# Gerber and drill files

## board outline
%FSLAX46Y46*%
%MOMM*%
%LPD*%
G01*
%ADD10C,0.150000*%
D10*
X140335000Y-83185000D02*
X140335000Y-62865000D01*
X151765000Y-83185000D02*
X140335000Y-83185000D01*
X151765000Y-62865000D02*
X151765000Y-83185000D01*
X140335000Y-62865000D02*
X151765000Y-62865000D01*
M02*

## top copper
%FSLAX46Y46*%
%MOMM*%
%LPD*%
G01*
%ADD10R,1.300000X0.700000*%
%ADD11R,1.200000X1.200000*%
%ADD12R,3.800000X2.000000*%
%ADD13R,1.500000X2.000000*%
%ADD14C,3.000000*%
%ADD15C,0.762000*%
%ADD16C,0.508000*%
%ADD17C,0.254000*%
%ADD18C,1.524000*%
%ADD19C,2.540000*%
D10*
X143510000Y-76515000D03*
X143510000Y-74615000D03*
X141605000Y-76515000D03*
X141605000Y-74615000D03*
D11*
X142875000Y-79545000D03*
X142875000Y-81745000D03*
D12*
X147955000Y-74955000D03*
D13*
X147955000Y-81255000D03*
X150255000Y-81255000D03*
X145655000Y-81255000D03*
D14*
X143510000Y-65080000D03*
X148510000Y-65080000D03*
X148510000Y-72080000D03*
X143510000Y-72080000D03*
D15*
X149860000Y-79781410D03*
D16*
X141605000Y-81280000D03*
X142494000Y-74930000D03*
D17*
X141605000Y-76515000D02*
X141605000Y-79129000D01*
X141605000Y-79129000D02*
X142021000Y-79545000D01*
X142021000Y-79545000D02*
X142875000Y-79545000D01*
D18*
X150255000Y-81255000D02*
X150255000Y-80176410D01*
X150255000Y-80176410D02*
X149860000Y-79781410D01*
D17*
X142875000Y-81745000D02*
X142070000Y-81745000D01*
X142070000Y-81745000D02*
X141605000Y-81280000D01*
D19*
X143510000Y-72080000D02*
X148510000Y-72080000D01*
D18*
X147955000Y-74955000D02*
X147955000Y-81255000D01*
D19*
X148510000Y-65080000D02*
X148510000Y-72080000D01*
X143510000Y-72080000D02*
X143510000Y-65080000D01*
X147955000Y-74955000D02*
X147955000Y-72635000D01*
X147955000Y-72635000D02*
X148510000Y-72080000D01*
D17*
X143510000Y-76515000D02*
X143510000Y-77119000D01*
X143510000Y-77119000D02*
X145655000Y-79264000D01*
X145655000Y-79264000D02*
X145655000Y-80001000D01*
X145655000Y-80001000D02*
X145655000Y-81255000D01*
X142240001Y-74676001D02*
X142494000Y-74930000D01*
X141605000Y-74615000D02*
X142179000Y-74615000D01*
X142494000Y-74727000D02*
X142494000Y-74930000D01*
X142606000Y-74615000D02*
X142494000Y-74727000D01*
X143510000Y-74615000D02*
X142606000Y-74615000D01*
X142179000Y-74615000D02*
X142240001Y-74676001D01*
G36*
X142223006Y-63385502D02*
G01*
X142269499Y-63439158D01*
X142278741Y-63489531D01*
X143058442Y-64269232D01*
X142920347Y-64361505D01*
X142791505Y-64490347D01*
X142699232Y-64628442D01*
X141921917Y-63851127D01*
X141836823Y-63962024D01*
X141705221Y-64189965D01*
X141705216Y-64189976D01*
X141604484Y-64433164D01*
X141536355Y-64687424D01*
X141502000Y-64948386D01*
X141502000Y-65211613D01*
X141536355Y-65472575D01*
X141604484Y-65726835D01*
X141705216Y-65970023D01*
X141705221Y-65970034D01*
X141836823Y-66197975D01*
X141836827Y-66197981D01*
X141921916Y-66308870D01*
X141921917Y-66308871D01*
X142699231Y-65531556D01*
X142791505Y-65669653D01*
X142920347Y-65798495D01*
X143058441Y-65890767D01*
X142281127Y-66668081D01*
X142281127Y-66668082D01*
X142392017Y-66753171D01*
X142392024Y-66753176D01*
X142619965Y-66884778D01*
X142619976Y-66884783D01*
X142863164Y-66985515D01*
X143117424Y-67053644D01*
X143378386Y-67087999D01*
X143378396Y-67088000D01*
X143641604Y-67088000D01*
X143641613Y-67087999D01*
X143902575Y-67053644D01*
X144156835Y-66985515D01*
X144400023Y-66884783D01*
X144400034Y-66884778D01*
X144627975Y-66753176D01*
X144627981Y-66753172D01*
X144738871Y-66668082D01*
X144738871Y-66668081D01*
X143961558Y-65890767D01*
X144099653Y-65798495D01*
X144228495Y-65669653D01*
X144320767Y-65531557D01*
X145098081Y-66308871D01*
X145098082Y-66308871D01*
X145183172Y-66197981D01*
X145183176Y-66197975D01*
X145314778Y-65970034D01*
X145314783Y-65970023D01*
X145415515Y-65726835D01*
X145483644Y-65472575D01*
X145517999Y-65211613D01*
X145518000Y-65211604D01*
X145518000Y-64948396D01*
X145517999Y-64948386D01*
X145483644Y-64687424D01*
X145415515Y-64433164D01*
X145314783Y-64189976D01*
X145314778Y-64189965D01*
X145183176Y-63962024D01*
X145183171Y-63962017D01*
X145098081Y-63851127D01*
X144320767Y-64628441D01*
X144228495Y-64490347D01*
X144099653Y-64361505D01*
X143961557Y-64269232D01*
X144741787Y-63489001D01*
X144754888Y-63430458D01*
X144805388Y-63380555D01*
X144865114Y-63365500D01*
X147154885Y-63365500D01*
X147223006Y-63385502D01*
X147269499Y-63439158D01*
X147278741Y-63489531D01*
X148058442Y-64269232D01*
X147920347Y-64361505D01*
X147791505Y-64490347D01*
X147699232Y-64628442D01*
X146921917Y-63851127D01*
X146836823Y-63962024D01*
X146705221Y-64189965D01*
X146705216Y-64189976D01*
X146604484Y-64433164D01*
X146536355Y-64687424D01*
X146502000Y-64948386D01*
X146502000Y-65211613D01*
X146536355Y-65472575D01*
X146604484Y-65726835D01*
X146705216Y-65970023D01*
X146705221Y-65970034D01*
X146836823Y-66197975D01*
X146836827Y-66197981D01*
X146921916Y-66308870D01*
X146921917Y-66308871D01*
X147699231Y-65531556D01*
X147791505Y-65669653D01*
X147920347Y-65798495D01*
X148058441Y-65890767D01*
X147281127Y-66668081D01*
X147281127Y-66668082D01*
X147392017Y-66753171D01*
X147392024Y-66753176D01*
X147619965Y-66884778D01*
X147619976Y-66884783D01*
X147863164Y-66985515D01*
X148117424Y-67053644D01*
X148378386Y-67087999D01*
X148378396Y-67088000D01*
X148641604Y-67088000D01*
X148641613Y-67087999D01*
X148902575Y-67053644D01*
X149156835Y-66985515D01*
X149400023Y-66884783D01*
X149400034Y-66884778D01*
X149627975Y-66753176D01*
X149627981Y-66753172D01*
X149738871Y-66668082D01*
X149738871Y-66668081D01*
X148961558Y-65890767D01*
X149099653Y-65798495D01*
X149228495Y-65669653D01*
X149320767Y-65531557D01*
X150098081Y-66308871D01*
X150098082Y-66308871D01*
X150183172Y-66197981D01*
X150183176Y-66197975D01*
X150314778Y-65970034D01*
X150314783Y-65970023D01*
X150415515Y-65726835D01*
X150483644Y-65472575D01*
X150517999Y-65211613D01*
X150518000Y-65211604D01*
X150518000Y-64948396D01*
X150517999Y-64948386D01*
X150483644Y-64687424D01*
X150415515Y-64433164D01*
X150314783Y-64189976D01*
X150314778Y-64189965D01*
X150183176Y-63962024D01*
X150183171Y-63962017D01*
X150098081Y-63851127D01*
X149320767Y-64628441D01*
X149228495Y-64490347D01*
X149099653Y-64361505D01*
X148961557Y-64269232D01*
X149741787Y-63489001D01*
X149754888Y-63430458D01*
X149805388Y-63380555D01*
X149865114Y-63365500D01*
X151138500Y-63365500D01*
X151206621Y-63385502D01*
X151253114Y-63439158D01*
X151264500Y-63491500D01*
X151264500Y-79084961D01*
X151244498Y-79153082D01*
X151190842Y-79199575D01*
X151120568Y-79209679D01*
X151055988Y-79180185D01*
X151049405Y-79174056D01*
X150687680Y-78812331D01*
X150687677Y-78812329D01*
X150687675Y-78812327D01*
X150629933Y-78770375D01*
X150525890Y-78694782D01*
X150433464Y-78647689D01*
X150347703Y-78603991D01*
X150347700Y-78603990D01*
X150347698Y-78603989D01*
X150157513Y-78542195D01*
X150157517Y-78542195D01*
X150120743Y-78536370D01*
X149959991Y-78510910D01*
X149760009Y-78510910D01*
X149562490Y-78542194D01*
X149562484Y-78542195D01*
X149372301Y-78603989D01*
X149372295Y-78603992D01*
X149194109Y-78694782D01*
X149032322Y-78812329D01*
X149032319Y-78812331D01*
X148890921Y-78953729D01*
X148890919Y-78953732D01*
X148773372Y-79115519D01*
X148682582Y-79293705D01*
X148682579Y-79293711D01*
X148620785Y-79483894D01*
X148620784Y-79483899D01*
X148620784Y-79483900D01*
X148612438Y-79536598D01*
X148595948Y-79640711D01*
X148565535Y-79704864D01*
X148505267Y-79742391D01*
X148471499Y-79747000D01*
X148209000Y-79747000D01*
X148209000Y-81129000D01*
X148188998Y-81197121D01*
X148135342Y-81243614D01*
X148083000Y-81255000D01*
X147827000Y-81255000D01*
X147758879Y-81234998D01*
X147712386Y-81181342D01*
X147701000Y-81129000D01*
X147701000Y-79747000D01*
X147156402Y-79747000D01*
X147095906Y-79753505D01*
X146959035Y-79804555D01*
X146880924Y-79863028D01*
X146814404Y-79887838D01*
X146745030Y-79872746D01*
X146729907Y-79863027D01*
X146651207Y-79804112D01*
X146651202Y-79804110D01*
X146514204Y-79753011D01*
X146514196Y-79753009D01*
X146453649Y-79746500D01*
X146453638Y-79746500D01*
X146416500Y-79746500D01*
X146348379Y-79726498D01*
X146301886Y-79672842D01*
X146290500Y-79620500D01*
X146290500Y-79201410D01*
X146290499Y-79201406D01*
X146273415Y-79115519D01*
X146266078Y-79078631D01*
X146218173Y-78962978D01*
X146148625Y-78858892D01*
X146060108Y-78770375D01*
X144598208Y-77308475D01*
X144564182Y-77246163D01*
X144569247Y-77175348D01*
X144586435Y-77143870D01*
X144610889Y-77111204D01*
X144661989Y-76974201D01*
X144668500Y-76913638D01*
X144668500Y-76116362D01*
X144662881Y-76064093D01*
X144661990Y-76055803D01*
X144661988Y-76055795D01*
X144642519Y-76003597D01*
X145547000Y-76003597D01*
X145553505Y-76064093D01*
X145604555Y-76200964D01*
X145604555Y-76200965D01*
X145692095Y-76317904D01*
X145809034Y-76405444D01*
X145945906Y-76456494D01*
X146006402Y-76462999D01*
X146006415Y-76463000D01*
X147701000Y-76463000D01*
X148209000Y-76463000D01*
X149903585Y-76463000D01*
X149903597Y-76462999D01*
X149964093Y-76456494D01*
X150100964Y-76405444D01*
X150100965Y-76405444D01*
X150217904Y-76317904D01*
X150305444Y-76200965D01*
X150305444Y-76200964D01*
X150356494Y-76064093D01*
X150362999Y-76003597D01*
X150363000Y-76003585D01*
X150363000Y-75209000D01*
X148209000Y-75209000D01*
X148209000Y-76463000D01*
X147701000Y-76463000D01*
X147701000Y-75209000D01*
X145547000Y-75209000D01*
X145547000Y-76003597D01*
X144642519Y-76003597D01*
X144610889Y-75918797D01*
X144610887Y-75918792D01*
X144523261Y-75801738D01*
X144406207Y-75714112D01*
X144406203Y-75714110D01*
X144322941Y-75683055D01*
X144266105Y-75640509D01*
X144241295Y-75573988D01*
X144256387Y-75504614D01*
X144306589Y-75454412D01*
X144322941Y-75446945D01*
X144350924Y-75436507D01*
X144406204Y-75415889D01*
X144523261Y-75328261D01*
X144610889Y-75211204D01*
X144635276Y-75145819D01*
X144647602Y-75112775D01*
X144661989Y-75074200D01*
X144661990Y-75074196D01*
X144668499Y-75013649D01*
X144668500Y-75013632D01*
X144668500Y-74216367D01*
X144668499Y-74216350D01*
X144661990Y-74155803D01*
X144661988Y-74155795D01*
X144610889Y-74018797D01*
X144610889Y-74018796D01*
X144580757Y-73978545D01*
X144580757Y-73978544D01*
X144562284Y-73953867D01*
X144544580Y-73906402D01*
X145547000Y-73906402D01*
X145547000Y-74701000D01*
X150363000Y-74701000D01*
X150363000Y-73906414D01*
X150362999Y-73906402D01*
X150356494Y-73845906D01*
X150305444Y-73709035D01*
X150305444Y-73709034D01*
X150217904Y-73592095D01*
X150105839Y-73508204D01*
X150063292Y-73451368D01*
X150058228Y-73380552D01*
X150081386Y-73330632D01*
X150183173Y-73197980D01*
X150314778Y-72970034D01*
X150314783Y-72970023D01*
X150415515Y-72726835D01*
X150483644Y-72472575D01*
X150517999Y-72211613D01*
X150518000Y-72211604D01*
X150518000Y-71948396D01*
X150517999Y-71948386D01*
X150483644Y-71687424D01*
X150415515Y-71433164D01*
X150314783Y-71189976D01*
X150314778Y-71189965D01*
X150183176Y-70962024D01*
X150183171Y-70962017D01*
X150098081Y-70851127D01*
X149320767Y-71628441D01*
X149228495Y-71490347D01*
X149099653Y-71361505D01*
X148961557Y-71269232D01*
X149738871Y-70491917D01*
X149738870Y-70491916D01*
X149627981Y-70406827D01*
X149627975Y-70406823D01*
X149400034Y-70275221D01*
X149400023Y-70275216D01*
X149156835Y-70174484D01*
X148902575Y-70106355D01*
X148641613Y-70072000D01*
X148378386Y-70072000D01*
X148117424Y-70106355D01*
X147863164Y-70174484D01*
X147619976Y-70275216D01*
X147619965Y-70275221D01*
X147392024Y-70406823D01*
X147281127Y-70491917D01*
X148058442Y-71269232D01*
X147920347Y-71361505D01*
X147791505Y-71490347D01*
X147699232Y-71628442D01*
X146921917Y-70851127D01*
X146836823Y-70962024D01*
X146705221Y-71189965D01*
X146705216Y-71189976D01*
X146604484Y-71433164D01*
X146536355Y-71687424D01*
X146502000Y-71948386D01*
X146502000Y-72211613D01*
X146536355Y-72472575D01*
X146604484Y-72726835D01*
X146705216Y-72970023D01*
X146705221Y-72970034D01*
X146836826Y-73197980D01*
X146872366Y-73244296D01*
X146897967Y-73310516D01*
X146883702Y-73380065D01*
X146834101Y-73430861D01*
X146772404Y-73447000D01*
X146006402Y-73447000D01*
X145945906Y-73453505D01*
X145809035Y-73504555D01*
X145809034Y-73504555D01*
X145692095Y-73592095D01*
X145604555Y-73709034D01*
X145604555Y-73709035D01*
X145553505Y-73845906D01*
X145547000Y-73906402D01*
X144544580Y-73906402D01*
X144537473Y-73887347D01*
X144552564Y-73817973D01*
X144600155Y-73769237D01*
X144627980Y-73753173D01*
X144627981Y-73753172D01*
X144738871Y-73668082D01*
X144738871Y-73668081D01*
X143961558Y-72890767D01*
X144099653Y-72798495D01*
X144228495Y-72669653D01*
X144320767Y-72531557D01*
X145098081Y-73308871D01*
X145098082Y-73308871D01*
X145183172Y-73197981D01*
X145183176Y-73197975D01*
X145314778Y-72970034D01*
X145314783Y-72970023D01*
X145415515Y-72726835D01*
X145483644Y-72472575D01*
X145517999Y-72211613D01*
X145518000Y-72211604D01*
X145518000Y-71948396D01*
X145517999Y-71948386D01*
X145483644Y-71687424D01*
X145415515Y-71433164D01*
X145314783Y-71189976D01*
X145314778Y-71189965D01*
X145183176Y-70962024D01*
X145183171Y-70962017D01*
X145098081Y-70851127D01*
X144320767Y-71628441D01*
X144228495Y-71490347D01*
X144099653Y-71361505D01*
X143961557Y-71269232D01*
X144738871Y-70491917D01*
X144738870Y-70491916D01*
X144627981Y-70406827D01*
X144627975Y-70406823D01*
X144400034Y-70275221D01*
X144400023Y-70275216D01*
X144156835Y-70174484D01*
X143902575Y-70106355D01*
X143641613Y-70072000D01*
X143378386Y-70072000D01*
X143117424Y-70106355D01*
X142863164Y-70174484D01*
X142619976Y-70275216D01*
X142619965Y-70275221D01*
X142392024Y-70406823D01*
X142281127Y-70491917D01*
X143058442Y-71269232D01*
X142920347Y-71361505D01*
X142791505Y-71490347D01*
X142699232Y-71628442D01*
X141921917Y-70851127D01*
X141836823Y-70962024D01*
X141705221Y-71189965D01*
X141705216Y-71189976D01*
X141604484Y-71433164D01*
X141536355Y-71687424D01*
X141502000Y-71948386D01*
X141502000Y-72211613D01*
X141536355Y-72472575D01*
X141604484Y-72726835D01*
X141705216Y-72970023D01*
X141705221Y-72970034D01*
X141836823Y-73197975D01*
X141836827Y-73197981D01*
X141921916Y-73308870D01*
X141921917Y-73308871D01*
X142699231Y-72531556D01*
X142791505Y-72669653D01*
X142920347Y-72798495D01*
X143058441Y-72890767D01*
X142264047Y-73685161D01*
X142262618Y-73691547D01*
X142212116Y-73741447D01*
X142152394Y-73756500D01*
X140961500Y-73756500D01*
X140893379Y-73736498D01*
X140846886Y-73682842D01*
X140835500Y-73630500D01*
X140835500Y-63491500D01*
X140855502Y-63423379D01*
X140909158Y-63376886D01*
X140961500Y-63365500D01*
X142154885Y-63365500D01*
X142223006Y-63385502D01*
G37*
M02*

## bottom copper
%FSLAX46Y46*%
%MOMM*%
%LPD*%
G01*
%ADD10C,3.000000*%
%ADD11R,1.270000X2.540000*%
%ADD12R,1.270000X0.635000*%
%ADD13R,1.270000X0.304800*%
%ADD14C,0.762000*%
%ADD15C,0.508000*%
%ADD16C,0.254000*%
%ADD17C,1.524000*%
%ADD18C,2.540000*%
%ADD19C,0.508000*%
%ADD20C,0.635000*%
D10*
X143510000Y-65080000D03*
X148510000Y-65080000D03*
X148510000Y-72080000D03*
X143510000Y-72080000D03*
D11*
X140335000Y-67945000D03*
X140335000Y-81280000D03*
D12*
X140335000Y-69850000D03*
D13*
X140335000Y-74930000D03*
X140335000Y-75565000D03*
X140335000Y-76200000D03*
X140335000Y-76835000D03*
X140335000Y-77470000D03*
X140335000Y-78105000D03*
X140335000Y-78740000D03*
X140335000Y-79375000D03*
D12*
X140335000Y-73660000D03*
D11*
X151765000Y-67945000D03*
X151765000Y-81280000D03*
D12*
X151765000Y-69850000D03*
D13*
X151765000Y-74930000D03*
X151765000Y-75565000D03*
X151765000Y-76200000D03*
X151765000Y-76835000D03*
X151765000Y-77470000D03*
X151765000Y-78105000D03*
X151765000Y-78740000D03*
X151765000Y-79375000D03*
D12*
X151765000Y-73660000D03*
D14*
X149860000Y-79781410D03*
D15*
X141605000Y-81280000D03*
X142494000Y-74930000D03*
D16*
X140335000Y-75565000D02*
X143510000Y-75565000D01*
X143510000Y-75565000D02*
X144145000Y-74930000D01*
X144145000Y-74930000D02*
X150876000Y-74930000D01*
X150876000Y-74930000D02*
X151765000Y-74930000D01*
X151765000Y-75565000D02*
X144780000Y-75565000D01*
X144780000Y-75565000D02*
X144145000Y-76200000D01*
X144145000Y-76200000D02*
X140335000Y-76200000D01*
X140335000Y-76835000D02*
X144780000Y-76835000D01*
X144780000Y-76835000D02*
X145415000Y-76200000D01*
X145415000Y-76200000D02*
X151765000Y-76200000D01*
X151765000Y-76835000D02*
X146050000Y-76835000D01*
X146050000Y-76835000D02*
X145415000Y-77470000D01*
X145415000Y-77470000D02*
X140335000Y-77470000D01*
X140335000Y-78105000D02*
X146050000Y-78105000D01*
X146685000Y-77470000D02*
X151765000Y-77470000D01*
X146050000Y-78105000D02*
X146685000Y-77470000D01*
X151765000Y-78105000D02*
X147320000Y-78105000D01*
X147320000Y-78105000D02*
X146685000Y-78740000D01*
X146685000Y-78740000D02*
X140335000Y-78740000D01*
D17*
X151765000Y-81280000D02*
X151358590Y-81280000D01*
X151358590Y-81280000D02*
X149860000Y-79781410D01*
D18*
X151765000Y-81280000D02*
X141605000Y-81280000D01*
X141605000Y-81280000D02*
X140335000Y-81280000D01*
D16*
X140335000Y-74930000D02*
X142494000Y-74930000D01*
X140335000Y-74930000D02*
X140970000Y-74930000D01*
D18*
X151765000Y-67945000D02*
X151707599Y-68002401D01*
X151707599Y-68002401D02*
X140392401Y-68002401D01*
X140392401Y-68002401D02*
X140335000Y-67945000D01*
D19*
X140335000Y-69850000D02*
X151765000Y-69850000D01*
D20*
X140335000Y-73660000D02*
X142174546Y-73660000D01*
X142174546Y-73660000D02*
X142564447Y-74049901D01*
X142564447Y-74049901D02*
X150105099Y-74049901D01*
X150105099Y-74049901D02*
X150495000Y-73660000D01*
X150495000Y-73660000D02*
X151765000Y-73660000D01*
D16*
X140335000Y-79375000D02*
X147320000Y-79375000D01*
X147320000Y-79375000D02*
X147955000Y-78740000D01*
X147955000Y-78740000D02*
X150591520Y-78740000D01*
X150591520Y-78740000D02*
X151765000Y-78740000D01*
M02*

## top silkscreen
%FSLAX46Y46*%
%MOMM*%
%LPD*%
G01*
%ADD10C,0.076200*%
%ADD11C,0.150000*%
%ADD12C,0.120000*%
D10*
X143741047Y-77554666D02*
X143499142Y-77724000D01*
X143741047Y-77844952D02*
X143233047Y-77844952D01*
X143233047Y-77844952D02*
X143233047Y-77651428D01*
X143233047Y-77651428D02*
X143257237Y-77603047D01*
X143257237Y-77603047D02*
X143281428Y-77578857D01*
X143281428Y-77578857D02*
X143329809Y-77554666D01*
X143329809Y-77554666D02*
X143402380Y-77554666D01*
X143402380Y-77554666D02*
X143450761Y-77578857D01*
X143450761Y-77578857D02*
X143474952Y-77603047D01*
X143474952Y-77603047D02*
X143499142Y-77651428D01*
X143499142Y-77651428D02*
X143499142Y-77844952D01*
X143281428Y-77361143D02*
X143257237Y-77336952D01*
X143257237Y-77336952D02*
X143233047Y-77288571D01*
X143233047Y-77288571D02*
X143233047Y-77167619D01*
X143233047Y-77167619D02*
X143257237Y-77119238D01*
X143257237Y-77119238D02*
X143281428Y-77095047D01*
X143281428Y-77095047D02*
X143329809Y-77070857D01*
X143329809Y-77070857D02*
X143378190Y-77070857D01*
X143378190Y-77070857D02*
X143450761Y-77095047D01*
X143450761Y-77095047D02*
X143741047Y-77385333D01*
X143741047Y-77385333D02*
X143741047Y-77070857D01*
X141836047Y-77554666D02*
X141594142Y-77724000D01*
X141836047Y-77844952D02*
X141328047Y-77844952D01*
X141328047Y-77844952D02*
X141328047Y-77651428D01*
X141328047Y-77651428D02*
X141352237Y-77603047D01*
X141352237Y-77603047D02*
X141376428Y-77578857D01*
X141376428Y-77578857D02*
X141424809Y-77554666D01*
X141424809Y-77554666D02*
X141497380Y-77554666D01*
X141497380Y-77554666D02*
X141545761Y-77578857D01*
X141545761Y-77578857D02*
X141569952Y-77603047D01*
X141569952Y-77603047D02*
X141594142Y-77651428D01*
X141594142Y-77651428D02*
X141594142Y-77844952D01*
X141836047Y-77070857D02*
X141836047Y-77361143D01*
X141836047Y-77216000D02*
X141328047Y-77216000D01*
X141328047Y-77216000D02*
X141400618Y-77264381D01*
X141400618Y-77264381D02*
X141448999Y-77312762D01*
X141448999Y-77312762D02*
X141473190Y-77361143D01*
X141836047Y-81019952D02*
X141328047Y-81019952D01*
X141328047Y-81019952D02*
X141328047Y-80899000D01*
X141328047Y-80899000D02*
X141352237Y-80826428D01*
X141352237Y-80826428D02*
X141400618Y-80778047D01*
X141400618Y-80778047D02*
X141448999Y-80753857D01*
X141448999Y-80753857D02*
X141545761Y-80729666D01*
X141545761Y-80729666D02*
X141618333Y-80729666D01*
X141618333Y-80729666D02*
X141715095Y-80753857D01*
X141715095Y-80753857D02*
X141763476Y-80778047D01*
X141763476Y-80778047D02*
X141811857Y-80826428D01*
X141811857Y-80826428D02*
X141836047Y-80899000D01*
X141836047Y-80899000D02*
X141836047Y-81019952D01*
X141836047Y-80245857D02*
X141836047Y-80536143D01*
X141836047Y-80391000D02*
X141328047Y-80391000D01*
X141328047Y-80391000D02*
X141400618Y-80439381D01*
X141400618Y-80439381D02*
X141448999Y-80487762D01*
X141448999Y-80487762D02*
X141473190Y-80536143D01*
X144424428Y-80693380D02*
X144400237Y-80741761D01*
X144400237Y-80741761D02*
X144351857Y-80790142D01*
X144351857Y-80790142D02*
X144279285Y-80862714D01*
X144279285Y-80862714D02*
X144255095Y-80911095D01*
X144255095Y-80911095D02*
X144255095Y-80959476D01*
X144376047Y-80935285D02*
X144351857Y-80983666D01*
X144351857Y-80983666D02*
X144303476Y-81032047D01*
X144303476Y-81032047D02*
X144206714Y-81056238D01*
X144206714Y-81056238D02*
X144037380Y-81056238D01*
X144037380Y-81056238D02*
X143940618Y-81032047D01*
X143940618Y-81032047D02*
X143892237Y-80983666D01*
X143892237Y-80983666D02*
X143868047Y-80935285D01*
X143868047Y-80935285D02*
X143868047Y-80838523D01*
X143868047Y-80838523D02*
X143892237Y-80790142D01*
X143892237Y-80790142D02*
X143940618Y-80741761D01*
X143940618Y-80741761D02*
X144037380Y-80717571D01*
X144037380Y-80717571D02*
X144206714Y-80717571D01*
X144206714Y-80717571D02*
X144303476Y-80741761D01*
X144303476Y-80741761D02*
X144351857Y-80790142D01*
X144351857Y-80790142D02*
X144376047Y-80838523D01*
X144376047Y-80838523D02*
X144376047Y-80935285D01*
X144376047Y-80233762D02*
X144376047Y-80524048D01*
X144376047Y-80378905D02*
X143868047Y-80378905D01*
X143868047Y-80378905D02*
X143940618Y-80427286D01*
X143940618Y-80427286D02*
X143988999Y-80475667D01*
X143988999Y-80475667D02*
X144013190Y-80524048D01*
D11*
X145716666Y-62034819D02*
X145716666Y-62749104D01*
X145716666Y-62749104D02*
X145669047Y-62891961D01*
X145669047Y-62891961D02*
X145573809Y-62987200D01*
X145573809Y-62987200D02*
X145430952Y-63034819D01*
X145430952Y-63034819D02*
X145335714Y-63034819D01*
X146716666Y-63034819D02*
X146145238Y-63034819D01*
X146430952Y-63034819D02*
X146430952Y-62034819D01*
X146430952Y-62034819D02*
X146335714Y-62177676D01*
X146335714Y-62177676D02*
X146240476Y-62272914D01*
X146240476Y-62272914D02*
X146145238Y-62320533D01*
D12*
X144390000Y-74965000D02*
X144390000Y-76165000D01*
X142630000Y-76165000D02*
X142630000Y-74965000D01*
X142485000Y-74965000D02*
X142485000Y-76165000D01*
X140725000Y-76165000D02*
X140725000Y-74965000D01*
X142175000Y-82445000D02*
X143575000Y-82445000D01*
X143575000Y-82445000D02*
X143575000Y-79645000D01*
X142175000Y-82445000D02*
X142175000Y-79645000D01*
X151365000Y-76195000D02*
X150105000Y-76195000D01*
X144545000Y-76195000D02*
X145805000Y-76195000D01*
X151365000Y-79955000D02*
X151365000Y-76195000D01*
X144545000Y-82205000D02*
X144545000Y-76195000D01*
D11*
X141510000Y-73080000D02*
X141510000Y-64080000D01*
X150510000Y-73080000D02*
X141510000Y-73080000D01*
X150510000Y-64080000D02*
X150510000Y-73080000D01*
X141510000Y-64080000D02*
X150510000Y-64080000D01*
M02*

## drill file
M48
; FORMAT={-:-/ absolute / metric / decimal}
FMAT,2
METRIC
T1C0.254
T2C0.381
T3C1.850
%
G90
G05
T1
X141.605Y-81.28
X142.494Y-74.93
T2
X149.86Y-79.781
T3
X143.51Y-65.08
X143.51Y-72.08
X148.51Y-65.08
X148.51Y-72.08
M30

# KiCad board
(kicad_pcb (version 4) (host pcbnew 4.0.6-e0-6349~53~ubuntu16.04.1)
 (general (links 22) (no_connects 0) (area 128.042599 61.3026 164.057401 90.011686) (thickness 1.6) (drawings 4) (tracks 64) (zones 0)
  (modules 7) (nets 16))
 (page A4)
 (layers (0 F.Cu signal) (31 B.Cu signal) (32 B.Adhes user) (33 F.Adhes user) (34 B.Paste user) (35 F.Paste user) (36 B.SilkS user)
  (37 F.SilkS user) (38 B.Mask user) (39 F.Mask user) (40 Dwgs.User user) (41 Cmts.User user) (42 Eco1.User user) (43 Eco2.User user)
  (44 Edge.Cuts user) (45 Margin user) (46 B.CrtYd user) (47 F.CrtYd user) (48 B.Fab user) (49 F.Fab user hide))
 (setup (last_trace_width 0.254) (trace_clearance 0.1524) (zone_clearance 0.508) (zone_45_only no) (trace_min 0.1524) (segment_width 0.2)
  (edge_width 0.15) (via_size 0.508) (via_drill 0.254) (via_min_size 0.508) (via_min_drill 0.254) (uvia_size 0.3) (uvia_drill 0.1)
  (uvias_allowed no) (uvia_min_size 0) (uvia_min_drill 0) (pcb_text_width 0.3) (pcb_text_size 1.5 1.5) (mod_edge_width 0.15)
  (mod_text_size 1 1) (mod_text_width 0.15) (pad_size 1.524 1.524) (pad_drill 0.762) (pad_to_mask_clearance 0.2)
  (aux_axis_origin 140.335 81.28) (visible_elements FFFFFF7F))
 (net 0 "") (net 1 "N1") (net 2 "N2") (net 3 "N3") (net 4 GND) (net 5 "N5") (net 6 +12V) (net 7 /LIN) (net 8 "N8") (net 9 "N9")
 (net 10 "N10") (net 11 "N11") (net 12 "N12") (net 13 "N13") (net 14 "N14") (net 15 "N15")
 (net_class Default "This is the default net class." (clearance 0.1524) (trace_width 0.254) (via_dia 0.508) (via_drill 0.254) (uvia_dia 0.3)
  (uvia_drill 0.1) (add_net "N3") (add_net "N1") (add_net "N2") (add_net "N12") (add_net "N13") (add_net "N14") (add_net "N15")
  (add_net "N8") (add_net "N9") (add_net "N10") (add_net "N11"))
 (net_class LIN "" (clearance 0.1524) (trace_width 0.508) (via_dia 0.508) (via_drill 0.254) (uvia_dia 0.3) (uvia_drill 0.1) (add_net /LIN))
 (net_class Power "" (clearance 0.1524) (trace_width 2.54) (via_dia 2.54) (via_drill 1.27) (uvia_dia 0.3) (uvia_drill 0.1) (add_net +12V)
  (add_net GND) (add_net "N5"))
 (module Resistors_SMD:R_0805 (layer F.Cu) (at 143.51 75.565 90)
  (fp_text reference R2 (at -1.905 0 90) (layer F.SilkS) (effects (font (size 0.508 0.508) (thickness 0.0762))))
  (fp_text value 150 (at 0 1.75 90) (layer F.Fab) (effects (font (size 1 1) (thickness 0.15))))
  (fp_line (start 0.6 0.88) (end -0.6 0.88) (layer F.SilkS) (width 0.12))
  (fp_line (start -0.6 -0.88) (end 0.6 -0.88) (layer F.SilkS) (width 0.12))
  (pad 1 smd rect (at -0.95 0 90) (size 0.7 1.3) (layers F.Cu F.Paste F.Mask) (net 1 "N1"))
  (pad 2 smd rect (at 0.95 0 90) (size 0.7 1.3) (layers F.Cu F.Paste F.Mask) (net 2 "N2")))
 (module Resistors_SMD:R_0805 (layer F.Cu) (at 141.605 75.565 90)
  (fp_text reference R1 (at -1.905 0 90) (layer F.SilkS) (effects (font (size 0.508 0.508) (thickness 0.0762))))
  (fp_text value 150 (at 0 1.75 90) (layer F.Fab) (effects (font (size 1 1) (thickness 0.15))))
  (fp_line (start 0.6 0.88) (end -0.6 0.88) (layer F.SilkS) (width 0.12))
  (fp_line (start -0.6 -0.88) (end 0.6 -0.88) (layer F.SilkS) (width 0.12))
  (pad 1 smd rect (at -0.95 0 90) (size 0.7 1.3) (layers F.Cu F.Paste F.Mask) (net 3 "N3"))
  (pad 2 smd rect (at 0.95 0 90) (size 0.7 1.3) (layers F.Cu F.Paste F.Mask) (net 2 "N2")))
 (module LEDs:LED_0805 (layer F.Cu) (at 142.875 80.645 90)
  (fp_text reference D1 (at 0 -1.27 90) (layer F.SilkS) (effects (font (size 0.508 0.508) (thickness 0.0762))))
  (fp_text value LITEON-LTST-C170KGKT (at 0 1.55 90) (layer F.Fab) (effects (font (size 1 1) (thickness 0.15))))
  (fp_line (start -1.8 -0.7) (end -1.8 0.7) (layer F.SilkS) (width 0.12))
  (fp_line (start -1.8 0.7) (end 1 0.7) (layer F.SilkS) (width 0.12))
  (fp_line (start -1.8 -0.7) (end 1 -0.7) (layer F.SilkS) (width 0.12))
  (pad 2 smd rect (at 1.1 0 270) (size 1.2 1.2) (layers F.Cu F.Paste F.Mask) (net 3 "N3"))
  (pad 1 smd rect (at -1.1 0 270) (size 1.2 1.2) (layers F.Cu F.Paste F.Mask) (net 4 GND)))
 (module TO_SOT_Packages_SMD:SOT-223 (layer F.Cu) (at 147.955 78.105 90)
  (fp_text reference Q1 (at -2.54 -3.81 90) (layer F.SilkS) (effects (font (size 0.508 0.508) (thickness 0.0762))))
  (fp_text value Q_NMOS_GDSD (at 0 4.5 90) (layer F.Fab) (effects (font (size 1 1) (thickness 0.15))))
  (fp_line (start 1.91 3.41) (end 1.91 2.15) (layer F.SilkS) (width 0.12))
  (fp_line (start 1.91 -3.41) (end 1.91 -2.15) (layer F.SilkS) (width 0.12))
  (fp_line (start -1.85 3.41) (end 1.91 3.41) (layer F.SilkS) (width 0.12))
  (fp_line (start -4.1 -3.41) (end 1.91 -3.41) (layer F.SilkS) (width 0.12))
  (pad 4 smd rect (at 3.15 0 90) (size 2 3.8) (layers F.Cu F.Paste F.Mask) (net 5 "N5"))
  (pad 2 smd rect (at -3.15 0 90) (size 2 1.5) (layers F.Cu F.Paste F.Mask) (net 5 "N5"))
  (pad 3 smd rect (at -3.15 2.3 90) (size 2 1.5) (layers F.Cu F.Paste F.Mask) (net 4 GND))
  (pad 1 smd rect (at -3.15 -2.3 90) (size 2 1.5) (layers F.Cu F.Paste F.Mask) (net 1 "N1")))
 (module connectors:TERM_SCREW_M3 (layer F.Cu) (at 146.01 68.58)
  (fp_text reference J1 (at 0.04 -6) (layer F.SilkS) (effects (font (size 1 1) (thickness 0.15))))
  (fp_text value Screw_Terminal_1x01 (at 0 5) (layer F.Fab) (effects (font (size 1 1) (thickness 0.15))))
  (fp_line (start -4.5 4.5) (end -4.5 -4.5) (layer F.SilkS) (width 0.15))
  (fp_line (start 4.5 4.5) (end -4.5 4.5) (layer F.SilkS) (width 0.15))
  (fp_line (start 4.5 -4.5) (end 4.5 4.5) (layer F.SilkS) (width 0.15))
  (fp_line (start -4.5 -4.5) (end 4.5 -4.5) (layer F.SilkS) (width 0.15))
  (pad 1 thru_hole circle (at -2.5 -3.5) (size 3 3) (drill 1.85) (layers *.Cu *.Mask) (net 5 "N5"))
  (pad 1 thru_hole circle (at 2.5 -3.5) (size 3 3) (drill 1.85) (layers *.Cu *.Mask) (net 5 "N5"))
  (pad 1 thru_hole circle (at 2.5 3.5) (size 3 3) (drill 1.85) (layers *.Cu *.Mask) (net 5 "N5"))
  (pad 1 thru_hole circle (at -2.5 3.5) (size 3 3) (drill 1.85) (layers *.Cu *.Mask) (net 5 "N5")))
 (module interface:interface (layer F.Cu) (at 140.335 63.5)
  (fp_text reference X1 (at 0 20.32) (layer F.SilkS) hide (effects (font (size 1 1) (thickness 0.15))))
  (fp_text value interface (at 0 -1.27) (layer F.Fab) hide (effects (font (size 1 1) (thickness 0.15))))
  (pad 1 smd rect (at 0 4.445) (size 1.27 2.54) (layers B.Cu) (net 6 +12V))
  (pad 2 smd rect (at 0 17.78) (size 1.27 2.54) (layers B.Cu) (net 4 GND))
  (pad 3 smd rect (at 0 6.35) (size 1.27 0.635) (layers B.Cu) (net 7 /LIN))
  (pad 5 smd rect (at 0 11.43) (size 1.27 0.3048) (layers B.Cu) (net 2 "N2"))
  (pad 6 smd rect (at 0 12.065) (size 1.27 0.3048) (layers B.Cu) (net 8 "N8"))
  (pad 7 smd rect (at 0 12.7) (size 1.27 0.3048) (layers B.Cu) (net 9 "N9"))
  (pad 8 smd rect (at 0 13.335) (size 1.27 0.3048) (layers B.Cu) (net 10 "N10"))
  (pad 9 smd rect (at 0 13.97) (size 1.27 0.3048) (layers B.Cu) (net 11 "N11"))
  (pad 10 smd rect (at 0 14.605) (size 1.27 0.3048) (layers B.Cu) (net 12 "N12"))
  (pad 11 smd rect (at 0 15.24) (size 1.27 0.3048) (layers B.Cu) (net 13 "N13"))
  (pad 12 smd rect (at 0 15.875) (size 1.27 0.3048) (layers B.Cu) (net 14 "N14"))
  (pad 4 smd rect (at 0 10.16) (size 1.27 0.635) (layers B.Cu) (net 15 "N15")))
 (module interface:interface (layer F.Cu) (at 151.765 63.5)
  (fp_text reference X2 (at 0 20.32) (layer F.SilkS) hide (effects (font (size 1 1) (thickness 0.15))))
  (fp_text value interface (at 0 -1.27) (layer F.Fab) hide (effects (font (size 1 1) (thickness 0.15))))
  (pad 1 smd rect (at 0 4.445) (size 1.27 2.54) (layers B.Cu) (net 6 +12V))
  (pad 2 smd rect (at 0 17.78) (size 1.27 2.54) (layers B.Cu) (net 4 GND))
  (pad 3 smd rect (at 0 6.35) (size 1.27 0.635) (layers B.Cu) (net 7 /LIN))
  (pad 5 smd rect (at 0 11.43) (size 1.27 0.3048) (layers B.Cu) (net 8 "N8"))
  (pad 6 smd rect (at 0 12.065) (size 1.27 0.3048) (layers B.Cu) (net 9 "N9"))
  (pad 7 smd rect (at 0 12.7) (size 1.27 0.3048) (layers B.Cu) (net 10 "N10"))
  (pad 8 smd rect (at 0 13.335) (size 1.27 0.3048) (layers B.Cu) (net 11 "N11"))
  (pad 9 smd rect (at 0 13.97) (size 1.27 0.3048) (layers B.Cu) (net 12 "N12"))
  (pad 10 smd rect (at 0 14.605) (size 1.27 0.3048) (layers B.Cu) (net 13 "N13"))
  (pad 11 smd rect (at 0 15.24) (size 1.27 0.3048) (layers B.Cu) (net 14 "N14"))
  (pad 12 smd rect (at 0 15.875) (size 1.27 0.3048) (layers B.Cu))
  (pad 4 smd rect (at 0 10.16) (size 1.27 0.635) (layers B.Cu) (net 15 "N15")))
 (gr_line (start 140.335 83.185) (end 140.335 62.865) (layer Edge.Cuts) (width 0.15))
 (gr_line (start 151.765 83.185) (end 140.335 83.185) (layer Edge.Cuts) (width 0.15))
 (gr_line (start 151.765 62.865) (end 151.765 83.185) (layer Edge.Cuts) (width 0.15))
 (gr_line (start 140.335 62.865) (end 151.765 62.865) (layer Edge.Cuts) (width 0.15))
 (segment (start 140.335 75.565) (end 143.51 75.565) (width 0.254) (layer B.Cu) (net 8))
 (segment (start 143.51 75.565) (end 144.145 74.93) (width 0.254) (layer B.Cu) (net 8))
 (segment (start 144.145 74.93) (end 150.876 74.93) (width 0.254) (layer B.Cu) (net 8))
 (segment (start 150.876 74.93) (end 151.765 74.93) (width 0.254) (layer B.Cu) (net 8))
 (segment (start 151.765 75.565) (end 144.78 75.565) (width 0.254) (layer B.Cu) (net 9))
 (segment (start 144.78 75.565) (end 144.145 76.2) (width 0.254) (layer B.Cu) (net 9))
 (segment (start 144.145 76.2) (end 140.335 76.2) (width 0.254) (layer B.Cu) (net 9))
 (segment (start 140.335 76.835) (end 144.78 76.835) (width 0.254) (layer B.Cu) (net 10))
 (segment (start 144.78 76.835) (end 145.415 76.2) (width 0.254) (layer B.Cu) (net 10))
 (segment (start 145.415 76.2) (end 151.765 76.2) (width 0.254) (layer B.Cu) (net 10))
 (segment (start 151.765 76.835) (end 146.05 76.835) (width 0.254) (layer B.Cu) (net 11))
 (segment (start 146.05 76.835) (end 145.415 77.47) (width 0.254) (layer B.Cu) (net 11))
 (segment (start 145.415 77.47) (end 140.335 77.47) (width 0.254) (layer B.Cu) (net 11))
 (segment (start 140.335 78.105) (end 146.05 78.105) (width 0.254) (layer B.Cu) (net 12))
 (segment (start 146.685 77.47) (end 151.765 77.47) (width 0.254) (layer B.Cu) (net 12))
 (segment (start 146.05 78.105) (end 146.685 77.47) (width 0.254) (layer B.Cu) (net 12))
 (segment (start 151.765 78.105) (end 147.32 78.105) (width 0.254) (layer B.Cu) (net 13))
 (segment (start 147.32 78.105) (end 146.685 78.74) (width 0.254) (layer B.Cu) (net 13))
 (segment (start 146.685 78.74) (end 140.335 78.74) (width 0.254) (layer B.Cu) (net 13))
 (segment (start 141.605 76.515) (end 141.605 79.129) (width 0.254) (layer F.Cu) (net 3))
 (segment (start 141.605 79.129) (end 142.021 79.545) (width 0.254) (layer F.Cu) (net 3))
 (segment (start 142.021 79.545) (end 142.875 79.545) (width 0.254) (layer F.Cu) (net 3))
 (segment (start 150.255 81.255) (end 150.255 80.17641) (width 1.524) (layer F.Cu) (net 4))
 (segment (start 150.255 80.17641) (end 149.86 79.78141) (width 1.524) (layer F.Cu) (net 4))
 (via (at 149.86 79.78141) (size 0.762) (drill 0.381) (layers F.Cu B.Cu) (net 4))
 (segment (start 151.765 81.28) (end 151.35859 81.28) (width 1.524) (layer B.Cu) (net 4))
 (segment (start 151.35859 81.28) (end 149.86 79.78141) (width 1.524) (layer B.Cu) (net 4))
 (segment (start 151.765 81.28) (end 141.605 81.28) (width 2.54) (layer B.Cu) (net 4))
 (segment (start 142.875 81.745) (end 142.07 81.745) (width 0.254) (layer F.Cu) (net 4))
 (segment (start 141.605 81.28) (end 140.335 81.28) (width 2.54) (layer B.Cu) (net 4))
 (segment (start 142.07 81.745) (end 141.605 81.28) (width 0.254) (layer F.Cu) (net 4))
 (via (at 141.605 81.28) (size 0.508) (drill 0.254) (layers F.Cu B.Cu) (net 4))
 (segment (start 143.51 72.08) (end 148.51 72.08) (width 2.54) (layer F.Cu) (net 5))
 (segment (start 147.955 74.955) (end 147.955 81.255) (width 1.524) (layer F.Cu) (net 5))
 (segment (start 148.51 65.08) (end 148.51 72.08) (width 2.54) (layer F.Cu) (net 5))
 (segment (start 143.51 72.08) (end 143.51 65.08) (width 2.54) (layer F.Cu) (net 5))
 (segment (start 147.955 74.955) (end 147.955 72.635) (width 2.54) (layer F.Cu) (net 5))
 (segment (start 147.955 72.635) (end 148.51 72.08) (width 2.54) (layer F.Cu) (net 5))
 (segment (start 143.51 76.515) (end 143.51 77.119) (width 0.254) (layer F.Cu) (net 1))
 (segment (start 143.51 77.119) (end 145.655 79.264) (width 0.254) (layer F.Cu) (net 1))
 (segment (start 145.655 79.264) (end 145.655 80.001) (width 0.254) (layer F.Cu) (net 1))
 (segment (start 145.655 80.001) (end 145.655 81.255) (width 0.254) (layer F.Cu) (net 1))
 (segment (start 142.240001 74.676001) (end 142.494 74.93) (width 0.254) (layer F.Cu) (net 2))
 (segment (start 141.605 74.615) (end 142.179 74.615) (width 0.254) (layer F.Cu) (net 2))
 (segment (start 142.494 74.727) (end 142.494 74.93) (width 0.254) (layer F.Cu) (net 2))
 (segment (start 142.606 74.615) (end 142.494 74.727) (width 0.254) (layer F.Cu) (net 2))
 (segment (start 143.51 74.615) (end 142.606 74.615) (width 0.254) (layer F.Cu) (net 2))
 (segment (start 142.179 74.615) (end 142.240001 74.676001) (width 0.254) (layer F.Cu) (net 2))
 (segment (start 140.335 74.93) (end 142.494 74.93) (width 0.254) (layer B.Cu) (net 2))
 (via (at 142.494 74.93) (size 0.508) (drill 0.254) (layers F.Cu B.Cu) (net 2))
 (segment (start 140.335 74.93) (end 140.97 74.93) (width 0.254) (layer B.Cu) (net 2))
 (segment (start 151.765 67.945) (end 151.707599 68.002401) (width 2.54) (layer B.Cu) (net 6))
 (segment (start 151.707599 68.002401) (end 140.392401 68.002401) (width 2.54) (layer B.Cu) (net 6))
 (segment (start 140.392401 68.002401) (end 140.335 67.945) (width 2.54) (layer B.Cu) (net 6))
 (segment (start 140.335 69.85) (end 151.765 69.85) (width 0.508) (layer B.Cu) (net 7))
 (segment (start 140.335 73.66) (end 142.174546 73.66) (width 0.635) (layer B.Cu) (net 15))
 (segment (start 142.174546 73.66) (end 142.564447 74.049901) (width 0.635) (layer B.Cu) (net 15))
 (segment (start 142.564447 74.049901) (end 150.105099 74.049901) (width 0.635) (layer B.Cu) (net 15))
 (segment (start 150.105099 74.049901) (end 150.495 73.66) (width 0.635) (layer B.Cu) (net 15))
 (segment (start 150.495 73.66) (end 151.765 73.66) (width 0.635) (layer B.Cu) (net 15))
 (segment (start 140.335 79.375) (end 147.32 79.375) (width 0.254) (layer B.Cu) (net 14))
 (segment (start 147.32 79.375) (end 147.955 78.74) (width 0.254) (layer B.Cu) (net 14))
 (segment (start 147.955 78.74) (end 150.59152 78.74) (width 0.254) (layer B.Cu) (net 14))
 (segment (start 150.59152 78.74) (end 151.765 78.74) (width 0.254) (layer B.Cu) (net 14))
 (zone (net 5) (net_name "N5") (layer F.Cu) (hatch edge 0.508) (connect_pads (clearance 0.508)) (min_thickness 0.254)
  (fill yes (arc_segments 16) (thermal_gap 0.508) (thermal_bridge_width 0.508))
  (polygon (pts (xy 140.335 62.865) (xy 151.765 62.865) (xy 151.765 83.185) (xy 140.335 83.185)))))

